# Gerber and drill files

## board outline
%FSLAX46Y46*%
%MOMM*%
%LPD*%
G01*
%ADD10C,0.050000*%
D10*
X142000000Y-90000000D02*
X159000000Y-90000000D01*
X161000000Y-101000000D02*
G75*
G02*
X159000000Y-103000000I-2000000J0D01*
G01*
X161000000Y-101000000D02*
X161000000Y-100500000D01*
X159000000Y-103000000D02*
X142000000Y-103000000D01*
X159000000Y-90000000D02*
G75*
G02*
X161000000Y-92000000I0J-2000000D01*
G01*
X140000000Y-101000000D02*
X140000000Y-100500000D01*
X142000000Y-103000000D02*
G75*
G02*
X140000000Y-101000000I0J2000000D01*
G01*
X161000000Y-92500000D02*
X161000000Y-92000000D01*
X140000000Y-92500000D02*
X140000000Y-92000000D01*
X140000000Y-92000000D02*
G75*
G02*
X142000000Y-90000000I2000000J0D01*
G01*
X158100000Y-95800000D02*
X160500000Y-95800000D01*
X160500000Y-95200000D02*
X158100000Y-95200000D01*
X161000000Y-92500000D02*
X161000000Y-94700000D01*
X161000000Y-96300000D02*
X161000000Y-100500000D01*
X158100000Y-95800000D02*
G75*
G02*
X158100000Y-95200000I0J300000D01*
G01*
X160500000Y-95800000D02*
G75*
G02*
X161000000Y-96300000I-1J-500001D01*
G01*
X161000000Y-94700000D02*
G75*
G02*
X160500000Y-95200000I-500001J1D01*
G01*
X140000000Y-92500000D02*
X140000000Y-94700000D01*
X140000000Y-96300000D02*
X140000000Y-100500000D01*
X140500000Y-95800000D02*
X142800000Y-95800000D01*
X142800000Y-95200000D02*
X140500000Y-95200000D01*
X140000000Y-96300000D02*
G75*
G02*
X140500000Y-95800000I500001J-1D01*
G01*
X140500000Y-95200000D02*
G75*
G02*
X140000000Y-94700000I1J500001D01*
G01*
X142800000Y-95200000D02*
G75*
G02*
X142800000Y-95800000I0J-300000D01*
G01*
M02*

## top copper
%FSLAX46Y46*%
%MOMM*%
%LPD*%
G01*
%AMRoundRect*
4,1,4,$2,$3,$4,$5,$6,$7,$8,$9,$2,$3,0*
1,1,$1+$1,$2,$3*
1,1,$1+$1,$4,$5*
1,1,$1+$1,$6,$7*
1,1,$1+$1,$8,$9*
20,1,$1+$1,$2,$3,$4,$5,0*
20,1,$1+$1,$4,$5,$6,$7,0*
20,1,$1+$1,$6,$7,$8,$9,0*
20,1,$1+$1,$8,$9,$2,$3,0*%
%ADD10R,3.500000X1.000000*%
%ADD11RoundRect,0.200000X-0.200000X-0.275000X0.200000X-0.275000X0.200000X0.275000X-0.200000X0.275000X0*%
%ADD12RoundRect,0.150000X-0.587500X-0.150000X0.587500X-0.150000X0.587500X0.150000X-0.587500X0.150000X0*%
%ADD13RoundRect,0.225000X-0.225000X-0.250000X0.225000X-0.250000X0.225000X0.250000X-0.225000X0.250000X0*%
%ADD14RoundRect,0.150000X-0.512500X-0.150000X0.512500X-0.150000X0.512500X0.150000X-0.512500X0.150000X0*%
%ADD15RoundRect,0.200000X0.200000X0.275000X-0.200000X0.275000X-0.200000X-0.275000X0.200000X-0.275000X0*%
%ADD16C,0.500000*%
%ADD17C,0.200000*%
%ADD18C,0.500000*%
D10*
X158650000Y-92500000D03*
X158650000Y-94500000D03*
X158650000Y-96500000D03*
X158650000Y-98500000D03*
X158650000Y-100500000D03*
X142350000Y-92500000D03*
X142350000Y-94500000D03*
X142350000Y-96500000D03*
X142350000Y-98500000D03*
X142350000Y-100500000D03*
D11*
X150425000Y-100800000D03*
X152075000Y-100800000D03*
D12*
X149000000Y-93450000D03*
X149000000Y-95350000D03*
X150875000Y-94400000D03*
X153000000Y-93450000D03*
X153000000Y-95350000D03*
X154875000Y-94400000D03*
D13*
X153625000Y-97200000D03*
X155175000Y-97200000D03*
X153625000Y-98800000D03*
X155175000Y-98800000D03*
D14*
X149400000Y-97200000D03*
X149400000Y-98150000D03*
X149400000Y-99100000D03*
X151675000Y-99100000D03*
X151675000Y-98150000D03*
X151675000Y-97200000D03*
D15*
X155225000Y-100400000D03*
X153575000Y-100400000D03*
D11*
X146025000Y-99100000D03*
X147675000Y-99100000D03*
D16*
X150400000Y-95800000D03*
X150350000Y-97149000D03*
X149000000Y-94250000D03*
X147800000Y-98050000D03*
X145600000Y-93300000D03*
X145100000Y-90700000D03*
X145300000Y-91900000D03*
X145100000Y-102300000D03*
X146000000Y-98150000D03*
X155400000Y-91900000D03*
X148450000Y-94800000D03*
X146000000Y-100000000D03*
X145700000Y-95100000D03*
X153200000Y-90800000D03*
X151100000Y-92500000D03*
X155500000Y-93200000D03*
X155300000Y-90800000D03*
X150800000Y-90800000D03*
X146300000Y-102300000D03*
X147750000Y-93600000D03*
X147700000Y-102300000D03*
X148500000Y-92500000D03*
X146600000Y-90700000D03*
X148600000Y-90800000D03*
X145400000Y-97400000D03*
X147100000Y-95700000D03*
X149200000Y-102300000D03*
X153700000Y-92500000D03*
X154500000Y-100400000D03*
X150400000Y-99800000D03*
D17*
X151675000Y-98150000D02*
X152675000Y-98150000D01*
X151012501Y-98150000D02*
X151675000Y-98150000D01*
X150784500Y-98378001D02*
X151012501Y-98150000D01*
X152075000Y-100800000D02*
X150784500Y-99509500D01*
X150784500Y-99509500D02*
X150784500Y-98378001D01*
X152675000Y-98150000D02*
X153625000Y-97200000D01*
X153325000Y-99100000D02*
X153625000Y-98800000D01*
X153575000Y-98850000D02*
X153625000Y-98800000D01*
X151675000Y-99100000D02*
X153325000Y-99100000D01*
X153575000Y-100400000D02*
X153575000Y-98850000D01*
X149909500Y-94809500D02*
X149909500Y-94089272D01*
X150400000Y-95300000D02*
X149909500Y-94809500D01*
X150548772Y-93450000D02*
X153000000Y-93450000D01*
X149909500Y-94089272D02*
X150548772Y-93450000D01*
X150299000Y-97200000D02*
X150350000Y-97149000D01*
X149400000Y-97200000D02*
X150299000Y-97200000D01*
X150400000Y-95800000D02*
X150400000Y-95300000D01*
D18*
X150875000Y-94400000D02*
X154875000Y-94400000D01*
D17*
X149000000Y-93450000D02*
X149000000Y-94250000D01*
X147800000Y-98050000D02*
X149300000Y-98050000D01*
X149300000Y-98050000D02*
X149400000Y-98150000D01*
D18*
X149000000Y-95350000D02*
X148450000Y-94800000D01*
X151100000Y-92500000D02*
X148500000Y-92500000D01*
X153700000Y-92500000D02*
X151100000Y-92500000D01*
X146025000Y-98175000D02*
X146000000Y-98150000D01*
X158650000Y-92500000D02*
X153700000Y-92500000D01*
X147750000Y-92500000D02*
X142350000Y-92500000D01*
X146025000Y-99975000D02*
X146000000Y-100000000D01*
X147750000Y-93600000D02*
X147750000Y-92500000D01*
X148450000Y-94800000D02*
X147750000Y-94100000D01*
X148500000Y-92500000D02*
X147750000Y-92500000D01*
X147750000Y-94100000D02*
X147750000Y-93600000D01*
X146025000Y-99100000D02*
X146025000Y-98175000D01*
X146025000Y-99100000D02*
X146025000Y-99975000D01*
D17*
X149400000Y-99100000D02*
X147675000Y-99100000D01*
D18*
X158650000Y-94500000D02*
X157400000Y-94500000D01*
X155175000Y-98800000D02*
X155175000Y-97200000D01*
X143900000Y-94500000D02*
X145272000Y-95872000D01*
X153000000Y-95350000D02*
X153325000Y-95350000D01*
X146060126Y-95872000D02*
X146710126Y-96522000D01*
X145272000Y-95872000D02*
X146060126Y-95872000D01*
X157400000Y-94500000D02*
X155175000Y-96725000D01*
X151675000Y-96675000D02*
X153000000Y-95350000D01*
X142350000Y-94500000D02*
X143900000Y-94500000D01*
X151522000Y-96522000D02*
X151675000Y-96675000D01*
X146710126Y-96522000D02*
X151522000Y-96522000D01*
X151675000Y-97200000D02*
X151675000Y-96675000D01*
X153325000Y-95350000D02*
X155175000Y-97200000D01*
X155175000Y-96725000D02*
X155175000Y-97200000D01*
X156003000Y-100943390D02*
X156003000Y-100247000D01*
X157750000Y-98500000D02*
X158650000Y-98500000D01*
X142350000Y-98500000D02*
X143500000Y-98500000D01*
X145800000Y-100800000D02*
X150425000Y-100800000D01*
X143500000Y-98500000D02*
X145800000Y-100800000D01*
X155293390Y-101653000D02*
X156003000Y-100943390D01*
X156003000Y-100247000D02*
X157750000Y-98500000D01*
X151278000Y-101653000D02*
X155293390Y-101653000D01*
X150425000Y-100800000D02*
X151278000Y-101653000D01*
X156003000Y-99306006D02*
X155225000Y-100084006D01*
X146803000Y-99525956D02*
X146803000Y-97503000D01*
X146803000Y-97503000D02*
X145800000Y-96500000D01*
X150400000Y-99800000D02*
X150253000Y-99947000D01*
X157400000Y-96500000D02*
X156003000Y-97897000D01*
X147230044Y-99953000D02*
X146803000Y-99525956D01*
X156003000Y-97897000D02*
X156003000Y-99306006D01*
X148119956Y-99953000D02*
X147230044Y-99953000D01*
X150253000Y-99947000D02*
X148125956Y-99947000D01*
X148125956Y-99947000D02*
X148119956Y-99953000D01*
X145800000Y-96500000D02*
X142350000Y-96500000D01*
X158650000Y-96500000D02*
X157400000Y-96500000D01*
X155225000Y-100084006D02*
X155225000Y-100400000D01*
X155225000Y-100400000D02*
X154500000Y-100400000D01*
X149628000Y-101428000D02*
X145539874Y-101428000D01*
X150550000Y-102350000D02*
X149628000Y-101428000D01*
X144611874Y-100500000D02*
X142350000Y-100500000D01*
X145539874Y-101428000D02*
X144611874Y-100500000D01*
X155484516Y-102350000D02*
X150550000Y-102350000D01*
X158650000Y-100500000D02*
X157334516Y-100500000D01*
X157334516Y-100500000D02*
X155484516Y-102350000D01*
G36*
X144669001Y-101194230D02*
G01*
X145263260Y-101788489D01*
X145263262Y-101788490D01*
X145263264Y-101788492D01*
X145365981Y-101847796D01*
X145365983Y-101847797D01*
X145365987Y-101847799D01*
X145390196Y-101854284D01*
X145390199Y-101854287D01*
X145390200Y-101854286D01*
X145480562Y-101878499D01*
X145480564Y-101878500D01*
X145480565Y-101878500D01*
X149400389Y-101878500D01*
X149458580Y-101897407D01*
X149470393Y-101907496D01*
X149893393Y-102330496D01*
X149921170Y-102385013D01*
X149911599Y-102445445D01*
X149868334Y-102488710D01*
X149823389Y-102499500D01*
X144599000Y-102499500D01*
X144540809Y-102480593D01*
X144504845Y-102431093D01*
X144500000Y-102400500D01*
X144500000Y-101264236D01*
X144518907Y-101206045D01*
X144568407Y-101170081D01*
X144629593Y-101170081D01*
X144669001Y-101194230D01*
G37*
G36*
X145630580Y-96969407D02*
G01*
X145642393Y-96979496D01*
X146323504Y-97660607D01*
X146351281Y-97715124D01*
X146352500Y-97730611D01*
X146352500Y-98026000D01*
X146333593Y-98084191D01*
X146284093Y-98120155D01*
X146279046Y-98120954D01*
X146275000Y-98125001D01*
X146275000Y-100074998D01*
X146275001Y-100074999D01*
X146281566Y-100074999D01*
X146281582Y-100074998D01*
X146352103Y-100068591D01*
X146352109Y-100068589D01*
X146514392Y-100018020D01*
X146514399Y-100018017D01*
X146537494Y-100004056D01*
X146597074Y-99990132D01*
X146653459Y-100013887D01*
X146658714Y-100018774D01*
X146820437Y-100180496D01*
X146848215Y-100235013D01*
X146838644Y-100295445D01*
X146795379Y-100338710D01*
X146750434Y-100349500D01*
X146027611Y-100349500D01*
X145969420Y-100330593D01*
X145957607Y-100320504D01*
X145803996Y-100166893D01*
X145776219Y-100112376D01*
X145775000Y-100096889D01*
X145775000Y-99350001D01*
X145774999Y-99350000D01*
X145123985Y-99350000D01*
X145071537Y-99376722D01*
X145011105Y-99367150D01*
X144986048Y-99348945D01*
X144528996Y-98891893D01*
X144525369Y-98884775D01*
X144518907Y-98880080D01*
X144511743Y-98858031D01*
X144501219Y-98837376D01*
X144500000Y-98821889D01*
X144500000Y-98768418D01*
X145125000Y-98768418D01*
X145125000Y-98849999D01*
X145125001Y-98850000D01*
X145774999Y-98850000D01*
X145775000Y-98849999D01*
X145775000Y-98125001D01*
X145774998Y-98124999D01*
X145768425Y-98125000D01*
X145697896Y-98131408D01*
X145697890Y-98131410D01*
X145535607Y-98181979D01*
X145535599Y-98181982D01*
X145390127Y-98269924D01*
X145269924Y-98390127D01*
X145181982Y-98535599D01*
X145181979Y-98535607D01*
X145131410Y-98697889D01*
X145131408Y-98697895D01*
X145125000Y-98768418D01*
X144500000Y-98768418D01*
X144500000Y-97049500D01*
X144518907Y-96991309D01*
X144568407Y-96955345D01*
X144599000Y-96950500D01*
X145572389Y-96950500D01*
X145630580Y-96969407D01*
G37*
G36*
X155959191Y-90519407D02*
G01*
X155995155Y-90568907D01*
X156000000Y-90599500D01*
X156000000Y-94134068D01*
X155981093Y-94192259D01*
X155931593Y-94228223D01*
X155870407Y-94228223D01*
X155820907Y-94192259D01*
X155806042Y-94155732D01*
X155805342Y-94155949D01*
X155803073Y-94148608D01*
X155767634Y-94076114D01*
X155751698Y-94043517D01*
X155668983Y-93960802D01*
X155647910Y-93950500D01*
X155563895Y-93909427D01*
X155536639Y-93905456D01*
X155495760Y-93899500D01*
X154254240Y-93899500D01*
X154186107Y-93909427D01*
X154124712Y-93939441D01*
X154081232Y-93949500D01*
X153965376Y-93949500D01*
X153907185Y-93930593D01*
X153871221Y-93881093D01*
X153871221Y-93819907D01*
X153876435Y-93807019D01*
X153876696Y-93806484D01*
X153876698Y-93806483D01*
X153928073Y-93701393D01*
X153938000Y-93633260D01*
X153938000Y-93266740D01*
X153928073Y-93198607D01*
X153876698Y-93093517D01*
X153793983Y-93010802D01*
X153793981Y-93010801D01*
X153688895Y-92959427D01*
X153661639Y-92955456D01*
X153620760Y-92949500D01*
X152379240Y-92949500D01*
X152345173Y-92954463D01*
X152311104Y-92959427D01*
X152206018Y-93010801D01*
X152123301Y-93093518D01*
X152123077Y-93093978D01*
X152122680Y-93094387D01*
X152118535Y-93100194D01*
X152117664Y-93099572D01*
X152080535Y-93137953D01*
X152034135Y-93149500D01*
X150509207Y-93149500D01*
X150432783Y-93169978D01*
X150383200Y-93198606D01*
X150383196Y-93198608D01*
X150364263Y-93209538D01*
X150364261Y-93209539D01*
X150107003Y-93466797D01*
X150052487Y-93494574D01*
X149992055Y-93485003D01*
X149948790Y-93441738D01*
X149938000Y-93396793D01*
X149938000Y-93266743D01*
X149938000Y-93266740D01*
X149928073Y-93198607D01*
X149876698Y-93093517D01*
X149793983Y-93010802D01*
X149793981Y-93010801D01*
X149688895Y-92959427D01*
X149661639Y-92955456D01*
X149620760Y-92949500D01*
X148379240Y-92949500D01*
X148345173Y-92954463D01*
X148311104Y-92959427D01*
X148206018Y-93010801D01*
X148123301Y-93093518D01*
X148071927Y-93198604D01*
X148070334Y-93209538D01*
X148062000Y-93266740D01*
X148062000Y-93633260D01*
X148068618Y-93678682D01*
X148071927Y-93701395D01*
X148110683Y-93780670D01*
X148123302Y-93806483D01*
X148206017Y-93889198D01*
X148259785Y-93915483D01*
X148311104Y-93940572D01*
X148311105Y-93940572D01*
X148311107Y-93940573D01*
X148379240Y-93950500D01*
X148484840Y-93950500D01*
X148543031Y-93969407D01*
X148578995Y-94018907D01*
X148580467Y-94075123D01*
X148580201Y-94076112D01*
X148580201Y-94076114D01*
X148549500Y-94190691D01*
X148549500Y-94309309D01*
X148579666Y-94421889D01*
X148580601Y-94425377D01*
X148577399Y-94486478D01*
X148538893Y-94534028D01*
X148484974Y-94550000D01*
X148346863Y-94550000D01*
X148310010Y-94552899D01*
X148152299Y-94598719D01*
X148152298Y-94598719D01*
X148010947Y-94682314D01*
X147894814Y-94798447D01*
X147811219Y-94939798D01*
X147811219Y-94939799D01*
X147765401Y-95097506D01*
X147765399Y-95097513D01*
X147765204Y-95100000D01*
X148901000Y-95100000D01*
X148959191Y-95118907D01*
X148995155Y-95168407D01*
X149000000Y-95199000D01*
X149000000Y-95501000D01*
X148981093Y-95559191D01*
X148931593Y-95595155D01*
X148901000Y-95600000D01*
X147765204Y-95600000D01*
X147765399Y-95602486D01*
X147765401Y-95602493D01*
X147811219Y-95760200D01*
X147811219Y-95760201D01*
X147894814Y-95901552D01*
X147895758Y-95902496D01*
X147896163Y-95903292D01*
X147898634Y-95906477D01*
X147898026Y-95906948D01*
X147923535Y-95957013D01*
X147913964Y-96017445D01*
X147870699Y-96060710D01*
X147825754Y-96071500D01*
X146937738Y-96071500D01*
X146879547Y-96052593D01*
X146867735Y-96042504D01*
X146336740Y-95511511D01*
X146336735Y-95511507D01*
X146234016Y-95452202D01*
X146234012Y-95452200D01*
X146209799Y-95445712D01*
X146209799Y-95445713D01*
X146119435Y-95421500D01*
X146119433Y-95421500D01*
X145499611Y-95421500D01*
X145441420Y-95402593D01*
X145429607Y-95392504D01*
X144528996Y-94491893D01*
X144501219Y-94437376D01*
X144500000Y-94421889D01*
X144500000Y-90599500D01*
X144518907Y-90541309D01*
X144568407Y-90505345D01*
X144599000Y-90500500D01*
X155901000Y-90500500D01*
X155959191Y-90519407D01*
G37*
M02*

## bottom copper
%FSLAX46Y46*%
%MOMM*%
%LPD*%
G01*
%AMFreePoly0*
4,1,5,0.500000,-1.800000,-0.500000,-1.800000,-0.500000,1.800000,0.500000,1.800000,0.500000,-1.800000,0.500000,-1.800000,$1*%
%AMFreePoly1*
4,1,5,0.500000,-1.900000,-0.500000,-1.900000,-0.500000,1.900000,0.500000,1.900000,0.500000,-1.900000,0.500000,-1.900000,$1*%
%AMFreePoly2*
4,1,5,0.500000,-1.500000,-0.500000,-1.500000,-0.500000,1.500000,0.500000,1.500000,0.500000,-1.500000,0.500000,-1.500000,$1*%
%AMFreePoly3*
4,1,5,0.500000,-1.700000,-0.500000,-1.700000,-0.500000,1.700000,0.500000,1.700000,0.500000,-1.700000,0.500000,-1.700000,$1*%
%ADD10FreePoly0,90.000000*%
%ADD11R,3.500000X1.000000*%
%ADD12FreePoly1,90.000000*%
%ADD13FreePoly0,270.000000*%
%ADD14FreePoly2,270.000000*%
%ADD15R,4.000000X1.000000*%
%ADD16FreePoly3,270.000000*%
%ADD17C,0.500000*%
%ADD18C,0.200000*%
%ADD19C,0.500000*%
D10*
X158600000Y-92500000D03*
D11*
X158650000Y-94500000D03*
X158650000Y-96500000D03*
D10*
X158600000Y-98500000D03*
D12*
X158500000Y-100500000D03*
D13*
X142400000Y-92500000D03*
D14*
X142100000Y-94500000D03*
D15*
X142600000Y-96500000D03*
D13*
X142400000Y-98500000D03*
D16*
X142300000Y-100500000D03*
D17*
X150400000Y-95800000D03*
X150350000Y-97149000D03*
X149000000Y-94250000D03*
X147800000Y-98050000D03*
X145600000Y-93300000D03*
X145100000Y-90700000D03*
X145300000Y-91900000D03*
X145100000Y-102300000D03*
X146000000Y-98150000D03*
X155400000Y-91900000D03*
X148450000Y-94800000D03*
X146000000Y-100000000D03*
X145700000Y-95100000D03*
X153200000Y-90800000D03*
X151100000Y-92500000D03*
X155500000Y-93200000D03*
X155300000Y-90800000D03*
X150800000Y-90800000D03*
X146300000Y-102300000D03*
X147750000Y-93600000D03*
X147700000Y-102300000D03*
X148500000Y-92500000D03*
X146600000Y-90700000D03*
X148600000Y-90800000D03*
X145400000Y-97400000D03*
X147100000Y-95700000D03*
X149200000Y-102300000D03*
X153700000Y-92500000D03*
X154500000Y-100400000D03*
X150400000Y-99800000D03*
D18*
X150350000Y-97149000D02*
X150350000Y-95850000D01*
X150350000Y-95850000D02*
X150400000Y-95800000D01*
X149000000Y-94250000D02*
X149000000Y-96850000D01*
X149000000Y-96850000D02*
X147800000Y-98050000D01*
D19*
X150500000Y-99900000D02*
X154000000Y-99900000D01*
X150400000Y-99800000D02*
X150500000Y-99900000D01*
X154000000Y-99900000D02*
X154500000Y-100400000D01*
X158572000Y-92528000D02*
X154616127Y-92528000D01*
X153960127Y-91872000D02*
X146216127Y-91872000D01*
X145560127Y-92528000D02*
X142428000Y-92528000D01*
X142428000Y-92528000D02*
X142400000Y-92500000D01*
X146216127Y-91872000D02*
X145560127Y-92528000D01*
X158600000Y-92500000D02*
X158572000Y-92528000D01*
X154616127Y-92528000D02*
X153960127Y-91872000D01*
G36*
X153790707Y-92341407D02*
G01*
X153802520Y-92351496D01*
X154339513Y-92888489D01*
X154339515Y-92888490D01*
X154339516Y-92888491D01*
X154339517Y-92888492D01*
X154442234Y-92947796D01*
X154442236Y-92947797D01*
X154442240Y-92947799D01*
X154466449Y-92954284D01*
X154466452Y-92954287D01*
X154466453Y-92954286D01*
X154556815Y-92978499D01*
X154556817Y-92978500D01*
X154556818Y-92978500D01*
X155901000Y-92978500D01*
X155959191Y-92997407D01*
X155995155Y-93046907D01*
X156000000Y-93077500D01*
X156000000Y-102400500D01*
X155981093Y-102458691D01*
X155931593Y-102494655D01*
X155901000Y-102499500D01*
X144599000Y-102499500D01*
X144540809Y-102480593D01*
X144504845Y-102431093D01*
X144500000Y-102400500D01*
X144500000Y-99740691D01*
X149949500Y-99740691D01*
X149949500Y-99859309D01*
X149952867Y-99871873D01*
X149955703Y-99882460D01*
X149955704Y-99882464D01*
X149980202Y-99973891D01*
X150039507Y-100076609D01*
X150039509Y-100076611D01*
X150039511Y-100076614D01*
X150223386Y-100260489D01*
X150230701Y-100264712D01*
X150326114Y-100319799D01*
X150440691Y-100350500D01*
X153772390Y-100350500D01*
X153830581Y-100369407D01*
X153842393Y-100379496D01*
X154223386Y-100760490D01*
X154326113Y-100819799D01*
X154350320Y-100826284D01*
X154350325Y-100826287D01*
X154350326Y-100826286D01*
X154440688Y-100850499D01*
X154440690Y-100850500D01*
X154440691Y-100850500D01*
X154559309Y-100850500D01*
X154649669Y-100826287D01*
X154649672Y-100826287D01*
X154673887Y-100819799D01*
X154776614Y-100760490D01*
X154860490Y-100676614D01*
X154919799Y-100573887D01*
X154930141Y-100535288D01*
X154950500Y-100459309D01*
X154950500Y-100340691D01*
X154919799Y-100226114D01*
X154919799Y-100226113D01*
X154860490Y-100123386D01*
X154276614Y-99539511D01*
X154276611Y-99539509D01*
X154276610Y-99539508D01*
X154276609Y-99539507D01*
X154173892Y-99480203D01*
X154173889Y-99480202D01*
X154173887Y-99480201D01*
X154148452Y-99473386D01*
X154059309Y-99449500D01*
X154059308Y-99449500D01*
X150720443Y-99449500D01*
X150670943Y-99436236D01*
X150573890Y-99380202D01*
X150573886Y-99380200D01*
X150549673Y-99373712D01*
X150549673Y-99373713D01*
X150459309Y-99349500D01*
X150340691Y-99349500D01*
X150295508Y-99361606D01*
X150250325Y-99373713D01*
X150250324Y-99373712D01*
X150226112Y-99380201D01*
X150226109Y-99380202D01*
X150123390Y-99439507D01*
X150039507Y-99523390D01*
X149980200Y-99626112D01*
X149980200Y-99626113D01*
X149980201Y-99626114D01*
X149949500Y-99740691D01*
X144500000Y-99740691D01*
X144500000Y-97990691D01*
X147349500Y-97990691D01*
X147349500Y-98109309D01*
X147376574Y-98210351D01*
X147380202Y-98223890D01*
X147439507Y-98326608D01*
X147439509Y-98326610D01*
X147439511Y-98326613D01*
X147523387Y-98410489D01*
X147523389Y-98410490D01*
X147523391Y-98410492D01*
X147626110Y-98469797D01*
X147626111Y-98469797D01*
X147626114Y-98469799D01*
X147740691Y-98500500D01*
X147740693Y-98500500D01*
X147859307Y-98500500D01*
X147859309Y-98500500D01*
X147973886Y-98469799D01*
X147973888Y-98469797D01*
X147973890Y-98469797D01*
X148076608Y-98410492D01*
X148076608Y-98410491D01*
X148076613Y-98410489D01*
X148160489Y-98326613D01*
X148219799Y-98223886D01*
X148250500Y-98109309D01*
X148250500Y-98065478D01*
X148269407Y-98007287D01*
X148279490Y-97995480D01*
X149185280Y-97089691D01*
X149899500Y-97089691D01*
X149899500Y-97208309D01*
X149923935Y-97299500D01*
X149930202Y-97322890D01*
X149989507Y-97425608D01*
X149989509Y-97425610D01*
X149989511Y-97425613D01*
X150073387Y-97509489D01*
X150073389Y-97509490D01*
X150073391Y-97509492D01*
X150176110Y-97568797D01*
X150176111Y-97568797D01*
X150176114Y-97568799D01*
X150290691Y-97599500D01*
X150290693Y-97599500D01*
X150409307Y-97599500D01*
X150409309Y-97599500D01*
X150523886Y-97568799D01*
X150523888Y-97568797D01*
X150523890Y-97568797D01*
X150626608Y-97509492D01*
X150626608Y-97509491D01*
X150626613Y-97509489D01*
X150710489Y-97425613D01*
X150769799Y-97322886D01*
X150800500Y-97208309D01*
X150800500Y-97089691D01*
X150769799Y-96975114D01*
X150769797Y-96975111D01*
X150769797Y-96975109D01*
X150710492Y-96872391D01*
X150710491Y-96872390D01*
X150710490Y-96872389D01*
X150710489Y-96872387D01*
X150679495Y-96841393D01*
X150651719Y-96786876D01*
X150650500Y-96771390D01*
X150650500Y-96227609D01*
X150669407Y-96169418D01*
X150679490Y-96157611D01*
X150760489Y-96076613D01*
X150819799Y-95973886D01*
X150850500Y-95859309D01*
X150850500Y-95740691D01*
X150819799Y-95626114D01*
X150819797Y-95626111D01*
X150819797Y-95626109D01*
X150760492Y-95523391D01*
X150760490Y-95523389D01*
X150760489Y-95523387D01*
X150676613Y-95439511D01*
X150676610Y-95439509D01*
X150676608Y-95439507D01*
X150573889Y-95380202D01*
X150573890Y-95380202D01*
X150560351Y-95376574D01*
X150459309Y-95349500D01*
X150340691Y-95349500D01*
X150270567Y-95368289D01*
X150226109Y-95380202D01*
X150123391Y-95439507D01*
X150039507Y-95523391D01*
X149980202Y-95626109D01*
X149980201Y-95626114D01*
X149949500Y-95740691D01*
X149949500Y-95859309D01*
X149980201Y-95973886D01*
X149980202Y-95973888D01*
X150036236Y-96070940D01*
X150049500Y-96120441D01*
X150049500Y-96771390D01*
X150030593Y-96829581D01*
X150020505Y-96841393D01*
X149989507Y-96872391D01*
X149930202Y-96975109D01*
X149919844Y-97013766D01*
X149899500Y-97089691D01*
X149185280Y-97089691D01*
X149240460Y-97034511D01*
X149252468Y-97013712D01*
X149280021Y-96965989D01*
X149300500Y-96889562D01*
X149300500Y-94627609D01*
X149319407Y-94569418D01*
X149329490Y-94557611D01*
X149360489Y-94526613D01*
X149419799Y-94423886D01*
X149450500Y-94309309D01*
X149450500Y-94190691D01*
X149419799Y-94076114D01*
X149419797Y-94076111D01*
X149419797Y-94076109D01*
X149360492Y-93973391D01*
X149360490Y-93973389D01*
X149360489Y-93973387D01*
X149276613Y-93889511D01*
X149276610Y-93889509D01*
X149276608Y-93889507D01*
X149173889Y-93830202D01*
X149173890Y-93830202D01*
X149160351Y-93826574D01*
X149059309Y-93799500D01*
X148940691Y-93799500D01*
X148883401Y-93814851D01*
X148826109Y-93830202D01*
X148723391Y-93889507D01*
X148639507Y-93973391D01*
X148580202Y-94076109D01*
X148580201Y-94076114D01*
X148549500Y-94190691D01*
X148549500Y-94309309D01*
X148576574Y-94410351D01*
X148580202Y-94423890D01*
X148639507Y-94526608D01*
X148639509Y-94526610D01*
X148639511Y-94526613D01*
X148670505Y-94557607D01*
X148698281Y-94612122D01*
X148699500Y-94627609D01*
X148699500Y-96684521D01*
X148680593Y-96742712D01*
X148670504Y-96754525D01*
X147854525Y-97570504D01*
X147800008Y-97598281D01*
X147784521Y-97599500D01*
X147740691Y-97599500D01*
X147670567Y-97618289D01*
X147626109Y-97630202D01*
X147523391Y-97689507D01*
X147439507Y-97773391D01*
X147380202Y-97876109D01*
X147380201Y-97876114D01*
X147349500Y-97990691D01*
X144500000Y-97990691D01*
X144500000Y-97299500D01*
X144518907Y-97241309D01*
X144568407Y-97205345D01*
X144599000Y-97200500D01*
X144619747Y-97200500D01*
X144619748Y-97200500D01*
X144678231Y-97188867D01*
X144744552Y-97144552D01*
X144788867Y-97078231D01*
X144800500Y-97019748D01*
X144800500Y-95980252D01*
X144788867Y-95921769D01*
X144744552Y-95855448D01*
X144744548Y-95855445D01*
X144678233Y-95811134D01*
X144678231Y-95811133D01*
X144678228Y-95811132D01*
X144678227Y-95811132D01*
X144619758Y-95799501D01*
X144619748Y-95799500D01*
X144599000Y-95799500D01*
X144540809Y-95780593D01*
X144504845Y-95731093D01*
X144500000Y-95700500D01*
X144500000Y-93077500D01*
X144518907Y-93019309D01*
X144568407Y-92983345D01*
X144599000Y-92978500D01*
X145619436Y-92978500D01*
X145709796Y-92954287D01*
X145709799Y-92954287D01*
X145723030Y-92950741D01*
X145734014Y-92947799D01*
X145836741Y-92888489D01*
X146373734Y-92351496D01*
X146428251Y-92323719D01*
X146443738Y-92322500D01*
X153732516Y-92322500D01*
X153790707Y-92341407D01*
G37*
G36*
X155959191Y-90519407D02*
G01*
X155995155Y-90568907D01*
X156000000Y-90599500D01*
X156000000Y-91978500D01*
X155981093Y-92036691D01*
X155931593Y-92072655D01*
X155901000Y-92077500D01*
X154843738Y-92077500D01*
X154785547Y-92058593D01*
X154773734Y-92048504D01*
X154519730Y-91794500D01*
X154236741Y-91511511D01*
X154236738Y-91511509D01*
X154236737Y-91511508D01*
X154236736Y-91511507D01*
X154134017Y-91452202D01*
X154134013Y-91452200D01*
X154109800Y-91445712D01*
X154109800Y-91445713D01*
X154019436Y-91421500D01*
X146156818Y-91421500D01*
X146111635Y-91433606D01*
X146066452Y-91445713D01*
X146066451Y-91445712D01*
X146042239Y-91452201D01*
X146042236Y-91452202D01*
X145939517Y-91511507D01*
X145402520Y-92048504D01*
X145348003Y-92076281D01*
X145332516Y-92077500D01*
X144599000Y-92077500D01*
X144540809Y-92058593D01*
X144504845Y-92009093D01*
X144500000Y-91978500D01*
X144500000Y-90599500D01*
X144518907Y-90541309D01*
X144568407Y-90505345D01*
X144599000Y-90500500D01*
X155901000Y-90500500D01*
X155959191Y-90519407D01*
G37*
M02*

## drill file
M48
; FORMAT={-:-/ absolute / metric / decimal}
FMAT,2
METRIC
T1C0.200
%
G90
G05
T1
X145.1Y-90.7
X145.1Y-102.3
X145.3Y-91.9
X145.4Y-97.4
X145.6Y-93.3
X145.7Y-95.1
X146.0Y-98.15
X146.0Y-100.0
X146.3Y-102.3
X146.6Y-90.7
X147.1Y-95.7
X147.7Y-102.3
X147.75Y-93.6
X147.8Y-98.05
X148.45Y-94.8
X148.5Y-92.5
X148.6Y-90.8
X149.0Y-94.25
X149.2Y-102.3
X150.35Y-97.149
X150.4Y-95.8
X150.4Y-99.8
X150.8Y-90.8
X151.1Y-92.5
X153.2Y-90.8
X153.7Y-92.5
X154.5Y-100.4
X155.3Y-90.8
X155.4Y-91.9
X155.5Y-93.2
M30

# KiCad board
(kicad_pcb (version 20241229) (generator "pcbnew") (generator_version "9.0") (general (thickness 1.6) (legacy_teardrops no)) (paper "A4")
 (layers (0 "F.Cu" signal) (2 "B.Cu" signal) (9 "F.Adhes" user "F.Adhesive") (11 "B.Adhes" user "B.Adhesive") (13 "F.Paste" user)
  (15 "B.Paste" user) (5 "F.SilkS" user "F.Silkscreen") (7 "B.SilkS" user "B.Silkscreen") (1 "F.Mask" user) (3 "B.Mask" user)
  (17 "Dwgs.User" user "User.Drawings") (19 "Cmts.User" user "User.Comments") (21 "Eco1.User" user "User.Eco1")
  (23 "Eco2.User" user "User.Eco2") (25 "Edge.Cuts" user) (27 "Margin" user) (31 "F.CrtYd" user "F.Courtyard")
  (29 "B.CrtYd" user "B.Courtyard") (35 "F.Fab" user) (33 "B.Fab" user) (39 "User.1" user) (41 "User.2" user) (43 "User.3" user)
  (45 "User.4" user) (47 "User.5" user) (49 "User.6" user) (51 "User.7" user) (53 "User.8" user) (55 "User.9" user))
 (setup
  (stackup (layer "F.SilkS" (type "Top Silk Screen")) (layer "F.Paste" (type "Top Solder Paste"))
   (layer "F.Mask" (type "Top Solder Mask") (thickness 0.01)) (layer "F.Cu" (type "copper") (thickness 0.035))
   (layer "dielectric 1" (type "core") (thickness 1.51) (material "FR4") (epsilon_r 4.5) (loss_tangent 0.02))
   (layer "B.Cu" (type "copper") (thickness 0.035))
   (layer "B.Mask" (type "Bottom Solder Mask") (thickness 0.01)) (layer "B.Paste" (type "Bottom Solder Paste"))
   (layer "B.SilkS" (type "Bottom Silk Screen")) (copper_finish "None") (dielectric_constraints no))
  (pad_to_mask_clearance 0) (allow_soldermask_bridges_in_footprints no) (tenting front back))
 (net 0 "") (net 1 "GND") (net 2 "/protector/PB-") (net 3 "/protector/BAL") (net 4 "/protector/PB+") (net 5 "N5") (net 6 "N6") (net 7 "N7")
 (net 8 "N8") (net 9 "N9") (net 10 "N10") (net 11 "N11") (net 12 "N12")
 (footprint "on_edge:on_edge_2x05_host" (layer "F.Cu") (at 161 96.5 -90)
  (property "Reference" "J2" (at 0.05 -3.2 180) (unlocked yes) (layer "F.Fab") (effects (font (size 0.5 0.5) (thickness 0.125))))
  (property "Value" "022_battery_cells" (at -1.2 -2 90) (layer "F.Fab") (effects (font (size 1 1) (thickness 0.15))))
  (fp_line (start -0.7 2.9) (end -0.7 0.5) (stroke (width 0.05) (type solid)) (layer "Edge.Cuts"))
  (fp_line (start -1.3 0.5) (end -1.3 2.9) (stroke (width 0.05) (type solid)) (layer "Edge.Cuts"))
  (fp_line (start -4 0) (end -1.8 0) (stroke (width 0.05) (type solid)) (layer "Edge.Cuts"))
  (fp_line (start -0.2 0) (end 4 0) (stroke (width 0.05) (type solid)) (layer "Edge.Cuts"))
  (fp_arc (start -0.7 2.9) (mid -1 3.2) (end -1.3 2.9) (stroke (width 0.05) (type solid)) (layer "Edge.Cuts"))
  (fp_arc (start -0.7 0.5) (mid -0.553553 0.146447) (end -0.2 0) (stroke (width 0.05) (type solid)) (layer "Edge.Cuts"))
  (fp_arc (start -1.8 0) (mid -1.446447 0.146447) (end -1.3 0.5) (stroke (width 0.05) (type solid)) (layer "Edge.Cuts"))
  (pad "1" smd rect (at -4 2.35 270) (size 1 3.5) (layers "F.Cu" "F.Mask") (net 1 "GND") (zone_connect 0))
  (pad "2" smd rect (at -2 2.35 270) (size 1 3.5) (layers "F.Cu" "F.Mask") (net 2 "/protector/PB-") (zone_connect 0))
  (pad "3" smd rect (at 0 2.35 270) (size 1 3.5) (layers "F.Cu" "F.Mask") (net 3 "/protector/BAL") (zone_connect 0))
  (pad "4" smd rect (at 2 2.35 270) (size 1 3.5) (layers "F.Cu" "F.Mask") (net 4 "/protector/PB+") (zone_connect 0))
  (pad "5" smd rect (at 4 2.35 270) (size 1 3.5) (layers "F.Cu" "F.Mask") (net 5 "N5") (zone_connect 0))
  (pad "6" smd custom (at -4 2.4 90) (size 1 3.6) (layers "B.Cu" "B.Mask") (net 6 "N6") (zone_connect 0)
   (options (clearance outline) (anchor rect)) (primitives))
  (pad "7" smd rect (at -2 2.35 90) (size 1 3.5) (layers "B.Cu" "B.Mask") (zone_connect 0))
  (pad "8" smd rect (at 0 2.35 90) (size 1 3.5) (layers "B.Cu" "B.Mask") (zone_connect 0))
  (pad "9" smd custom (at 2 2.4 90) (size 1 3.6) (layers "B.Cu" "B.Mask") (zone_connect 0) (options (clearance outline) (anchor rect))
   (primitives))
  (pad "10" smd custom (at 4 2.5 90) (size 1 3.8) (layers "B.Cu" "B.Mask") (zone_connect 0) (options (clearance outline) (anchor rect))
   (primitives))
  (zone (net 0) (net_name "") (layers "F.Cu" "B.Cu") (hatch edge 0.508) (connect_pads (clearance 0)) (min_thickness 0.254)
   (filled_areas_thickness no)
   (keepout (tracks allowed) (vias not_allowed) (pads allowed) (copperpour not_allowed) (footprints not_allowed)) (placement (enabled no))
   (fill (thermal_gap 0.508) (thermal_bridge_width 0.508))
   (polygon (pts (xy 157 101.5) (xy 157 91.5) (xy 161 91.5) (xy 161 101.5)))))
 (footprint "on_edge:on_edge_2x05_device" (layer "F.Cu") (at 140 96.5 -90)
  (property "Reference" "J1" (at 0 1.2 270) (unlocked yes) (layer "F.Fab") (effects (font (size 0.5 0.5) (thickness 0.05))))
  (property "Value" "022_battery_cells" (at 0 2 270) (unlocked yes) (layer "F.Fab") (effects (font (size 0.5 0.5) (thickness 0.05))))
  (fp_line (start -4 0) (end -1.8 0) (stroke (width 0.05) (type solid)) (layer "Edge.Cuts"))
  (fp_line (start -0.2 0) (end 4 0) (stroke (width 0.05) (type solid)) (layer "Edge.Cuts"))
  (fp_line (start -0.7 -0.5) (end -0.7 -2.8) (stroke (width 0.05) (type solid)) (layer "Edge.Cuts"))
  (fp_line (start -1.3 -2.8) (end -1.3 -0.5) (stroke (width 0.05) (type solid)) (layer "Edge.Cuts"))
  (fp_arc (start -0.2 0) (mid -0.553553 -0.146447) (end -0.7 -0.5) (stroke (width 0.05) (type solid)) (layer "Edge.Cuts"))
  (fp_arc (start -1.3 -0.5) (mid -1.446447 -0.146447) (end -1.8 0) (stroke (width 0.05) (type solid)) (layer "Edge.Cuts"))
  (fp_arc (start -1.3 -2.8) (mid -1 -3.1) (end -0.7 -2.8) (stroke (width 0.05) (type solid)) (layer "Edge.Cuts"))
  (pad "1" smd rect (at -4 -2.35 90) (size 1 3.5) (layers "F.Cu" "F.Mask") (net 1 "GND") (zone_connect 0))
  (pad "2" smd rect (at -2 -2.35 270) (size 1 3.5) (layers "F.Cu" "F.Mask") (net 2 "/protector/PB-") (zone_connect 0))
  (pad "3" smd rect (at 0 -2.35 270) (size 1 3.5) (layers "F.Cu" "F.Mask") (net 3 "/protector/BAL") (zone_connect 0))
  (pad "4" smd rect (at 2 -2.35 90) (size 1 3.5) (layers "F.Cu" "F.Mask") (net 4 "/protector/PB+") (zone_connect 0))
  (pad "5" smd rect (at 4 -2.35 90) (size 1 3.5) (layers "F.Cu" "F.Mask") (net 5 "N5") (zone_connect 0))
  (pad "6" smd custom (at -4 -2.4 270) (size 1 3.6) (layers "B.Cu" "B.Mask") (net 6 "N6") (zone_connect 0)
   (options (clearance outline) (anchor rect)) (primitives))
  (pad "7" smd custom (at -2 -2.1 270) (size 1 3) (layers "B.Cu" "B.Mask") (zone_connect 0) (options (clearance outline) (anchor rect))
   (primitives))
  (pad "8" smd rect (at 0 -2.6 270) (size 1 4) (layers "B.Cu" "B.Mask") (zone_connect 0))
  (pad "9" smd custom (at 2 -2.4 270) (size 1 3.6) (layers "B.Cu" "B.Mask") (zone_connect 0) (options (clearance outline) (anchor rect))
   (primitives))
  (pad "10" smd custom (at 4 -2.3 270) (size 1 3.4) (layers "B.Cu" "B.Mask") (zone_connect 0) (options (clearance outline) (anchor rect))
   (primitives))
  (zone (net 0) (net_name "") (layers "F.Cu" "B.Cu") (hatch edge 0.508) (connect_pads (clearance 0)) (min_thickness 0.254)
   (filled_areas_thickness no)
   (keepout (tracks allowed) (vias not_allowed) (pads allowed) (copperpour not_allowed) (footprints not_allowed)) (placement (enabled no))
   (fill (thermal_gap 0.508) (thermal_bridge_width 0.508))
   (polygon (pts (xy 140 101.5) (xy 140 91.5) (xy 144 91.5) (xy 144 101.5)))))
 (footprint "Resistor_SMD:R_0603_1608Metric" (layer "F.Cu") (at 151.25 100.8)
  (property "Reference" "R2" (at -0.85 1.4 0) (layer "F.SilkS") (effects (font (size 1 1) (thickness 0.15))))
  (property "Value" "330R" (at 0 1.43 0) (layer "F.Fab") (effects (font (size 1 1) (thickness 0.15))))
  (pad "1" smd roundrect (at -0.825 0) (size 0.8 0.95) (layers "F.Cu" "F.Mask" "F.Paste") (roundrect_rratio 0.25) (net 4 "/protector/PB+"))
  (pad "2" smd roundrect (at 0.825 0) (size 0.8 0.95) (layers "F.Cu" "F.Mask" "F.Paste") (roundrect_rratio 0.25) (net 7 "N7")))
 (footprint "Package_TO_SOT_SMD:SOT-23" (layer "F.Cu") (at 149.9375 94.4)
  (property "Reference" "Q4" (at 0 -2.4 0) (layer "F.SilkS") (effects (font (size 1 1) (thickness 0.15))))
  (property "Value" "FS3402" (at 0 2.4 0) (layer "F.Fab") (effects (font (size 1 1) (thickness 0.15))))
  (pad "1" smd roundrect (at -0.9375 -0.95) (size 1.475 0.6) (layers "F.Cu" "F.Mask" "F.Paste") (roundrect_rratio 0.25) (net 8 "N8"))
  (pad "2" smd roundrect (at -0.9375 0.95) (size 1.475 0.6) (layers "F.Cu" "F.Mask" "F.Paste") (roundrect_rratio 0.25) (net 1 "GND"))
  (pad "3" smd roundrect (at 0.9375 0) (size 1.475 0.6) (layers "F.Cu" "F.Mask" "F.Paste") (roundrect_rratio 0.25) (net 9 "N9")))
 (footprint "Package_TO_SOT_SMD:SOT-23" (layer "F.Cu") (at 153.9375 94.4)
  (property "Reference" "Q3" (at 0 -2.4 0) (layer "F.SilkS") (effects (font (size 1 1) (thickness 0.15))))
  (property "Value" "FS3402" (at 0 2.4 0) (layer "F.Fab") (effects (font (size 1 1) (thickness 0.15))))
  (pad "1" smd roundrect (at -0.9375 -0.95) (size 1.475 0.6) (layers "F.Cu" "F.Mask" "F.Paste") (roundrect_rratio 0.25) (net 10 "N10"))
  (pad "2" smd roundrect (at -0.9375 0.95) (size 1.475 0.6) (layers "F.Cu" "F.Mask" "F.Paste") (roundrect_rratio 0.25)
   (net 2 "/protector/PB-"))
  (pad "3" smd roundrect (at 0.9375 0) (size 1.475 0.6) (layers "F.Cu" "F.Mask" "F.Paste") (roundrect_rratio 0.25) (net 9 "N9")))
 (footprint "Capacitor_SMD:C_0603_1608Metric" (layer "F.Cu") (at 154.4 97.2)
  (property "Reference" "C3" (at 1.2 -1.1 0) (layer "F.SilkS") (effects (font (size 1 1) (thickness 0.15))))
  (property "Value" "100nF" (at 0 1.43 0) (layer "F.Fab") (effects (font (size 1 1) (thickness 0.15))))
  (pad "1" smd roundrect (at -0.775 0) (size 0.9 0.95) (layers "F.Cu" "F.Mask" "F.Paste") (roundrect_rratio 0.25) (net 7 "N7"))
  (pad "2" smd roundrect (at 0.775 0) (size 0.9 0.95) (layers "F.Cu" "F.Mask" "F.Paste") (roundrect_rratio 0.25) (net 2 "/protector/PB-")))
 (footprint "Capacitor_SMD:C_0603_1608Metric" (layer "F.Cu") (at 154.4 98.8)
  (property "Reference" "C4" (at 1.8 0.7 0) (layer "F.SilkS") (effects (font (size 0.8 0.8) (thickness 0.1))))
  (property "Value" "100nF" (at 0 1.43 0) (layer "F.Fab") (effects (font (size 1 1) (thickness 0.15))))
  (pad "1" smd roundrect (at -0.775 0) (size 0.9 0.95) (layers "F.Cu" "F.Mask" "F.Paste") (roundrect_rratio 0.25) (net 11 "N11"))
  (pad "2" smd roundrect (at 0.775 0) (size 0.9 0.95) (layers "F.Cu" "F.Mask" "F.Paste") (roundrect_rratio 0.25) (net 2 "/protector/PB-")))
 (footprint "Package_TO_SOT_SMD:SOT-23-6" (layer "F.Cu") (at 150.5375 98.15)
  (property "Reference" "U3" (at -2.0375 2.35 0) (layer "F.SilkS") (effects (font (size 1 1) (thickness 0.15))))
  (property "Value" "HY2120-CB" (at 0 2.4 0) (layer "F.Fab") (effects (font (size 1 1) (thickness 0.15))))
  (pad "1" smd roundrect (at -1.1375 -0.95) (size 1.325 0.6) (layers "F.Cu" "F.Mask" "F.Paste") (roundrect_rratio 0.25) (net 10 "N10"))
  (pad "2" smd roundrect (at -1.1375 0) (size 1.325 0.6) (layers "F.Cu" "F.Mask" "F.Paste") (roundrect_rratio 0.25) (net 8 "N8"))
  (pad "3" smd roundrect (at -1.1375 0.95) (size 1.325 0.6) (layers "F.Cu" "F.Mask" "F.Paste") (roundrect_rratio 0.25) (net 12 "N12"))
  (pad "4" smd roundrect (at 1.1375 0.95) (size 1.325 0.6) (layers "F.Cu" "F.Mask" "F.Paste") (roundrect_rratio 0.25) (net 11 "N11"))
  (pad "5" smd roundrect (at 1.1375 0) (size 1.325 0.6) (layers "F.Cu" "F.Mask" "F.Paste") (roundrect_rratio 0.25) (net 7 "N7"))
  (pad "6" smd roundrect (at 1.1375 -0.95) (size 1.325 0.6) (layers "F.Cu" "F.Mask" "F.Paste") (roundrect_rratio 0.25)
   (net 2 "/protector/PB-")))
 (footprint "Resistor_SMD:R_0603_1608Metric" (layer "F.Cu") (at 154.4 100.4 180)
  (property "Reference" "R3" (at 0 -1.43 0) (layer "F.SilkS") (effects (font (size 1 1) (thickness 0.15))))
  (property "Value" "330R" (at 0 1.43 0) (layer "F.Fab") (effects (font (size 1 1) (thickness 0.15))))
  (pad "1" smd roundrect (at -0.825 0 180) (size 0.8 0.95) (layers "F.Cu" "F.Mask" "F.Paste") (roundrect_rratio 0.25)
   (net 3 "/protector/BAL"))
  (pad "2" smd roundrect (at 0.825 0 180) (size 0.8 0.95) (layers "F.Cu" "F.Mask" "F.Paste") (roundrect_rratio 0.25) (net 11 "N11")))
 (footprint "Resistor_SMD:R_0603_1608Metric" (layer "F.Cu") (at 146.85 99.1)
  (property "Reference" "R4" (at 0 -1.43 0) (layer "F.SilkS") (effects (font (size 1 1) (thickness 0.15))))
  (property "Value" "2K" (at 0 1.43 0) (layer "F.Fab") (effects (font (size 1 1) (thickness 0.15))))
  (pad "1" smd roundrect (at -0.825 0) (size 0.8 0.95) (layers "F.Cu" "F.Mask" "F.Paste") (roundrect_rratio 0.25) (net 1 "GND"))
  (pad "2" smd roundrect (at 0.825 0) (size 0.8 0.95) (layers "F.Cu" "F.Mask" "F.Paste") (roundrect_rratio 0.25) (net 12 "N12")))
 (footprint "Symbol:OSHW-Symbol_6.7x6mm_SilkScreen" (layer "B.Cu") (at 149.175 95.9 180)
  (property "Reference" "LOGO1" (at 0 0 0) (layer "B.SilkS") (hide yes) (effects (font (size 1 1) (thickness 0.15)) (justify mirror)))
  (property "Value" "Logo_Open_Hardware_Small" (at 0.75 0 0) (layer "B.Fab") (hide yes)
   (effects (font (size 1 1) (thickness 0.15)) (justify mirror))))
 (gr_line (start 142 90) (end 159 90) (stroke (width 0.05) (type solid)) (layer "Edge.Cuts"))
 (gr_arc (start 161 101) (mid 160.414214 102.414214) (end 159 103) (stroke (width 0.05) (type solid)) (layer "Edge.Cuts"))
 (gr_line (start 161 101) (end 161 100.5) (stroke (width 0.05) (type solid)) (layer "Edge.Cuts"))
 (gr_line (start 159 103) (end 142 103) (stroke (width 0.05) (type solid)) (layer "Edge.Cuts"))
 (gr_arc (start 159 90) (mid 160.414214 90.585786) (end 161 92) (stroke (width 0.05) (type solid)) (layer "Edge.Cuts"))
 (gr_line (start 140 101) (end 140 100.5) (stroke (width 0.05) (type solid)) (layer "Edge.Cuts"))
 (gr_arc (start 142 103) (mid 140.585786 102.414214) (end 140 101) (stroke (width 0.05) (type solid)) (layer "Edge.Cuts"))
 (gr_line (start 161 92.5) (end 161 92) (stroke (width 0.05) (type solid)) (layer "Edge.Cuts"))
 (gr_line (start 140 92.5) (end 140 92) (stroke (width 0.05) (type solid)) (layer "Edge.Cuts"))
 (gr_arc (start 140 92) (mid 140.585786 90.585786) (end 142 90) (stroke (width 0.05) (type solid)) (layer "Edge.Cuts"))
 (segment (start 151.675 98.15) (end 152.675 98.15) (width 0.2) (layer "F.Cu") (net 7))
 (segment (start 151.012501 98.15) (end 151.675 98.15) (width 0.2) (layer "F.Cu") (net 7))
 (segment (start 150.7845 98.378001) (end 151.012501 98.15) (width 0.2) (layer "F.Cu") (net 7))
 (segment (start 152.075 100.8) (end 150.7845 99.5095) (width 0.2) (layer "F.Cu") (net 7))
 (segment (start 150.7845 99.5095) (end 150.7845 98.378001) (width 0.2) (layer "F.Cu") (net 7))
 (segment (start 152.675 98.15) (end 153.625 97.2) (width 0.2) (layer "F.Cu") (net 7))
 (segment (start 153.325 99.1) (end 153.625 98.8) (width 0.2) (layer "F.Cu") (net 11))
 (segment (start 153.575 98.85) (end 153.625 98.8) (width 0.2) (layer "F.Cu") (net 11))
 (segment (start 151.675 99.1) (end 153.325 99.1) (width 0.2) (layer "F.Cu") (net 11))
 (segment (start 153.575 100.4) (end 153.575 98.85) (width 0.2) (layer "F.Cu") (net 11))
 (segment (start 149.9095 94.8095) (end 149.9095 94.089272) (width 0.2) (layer "F.Cu") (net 10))
 (segment (start 150.4 95.3) (end 149.9095 94.8095) (width 0.2) (layer "F.Cu") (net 10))
 (segment (start 150.548772 93.45) (end 153 93.45) (width 0.2) (layer "F.Cu") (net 10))
 (segment (start 149.9095 94.089272) (end 150.548772 93.45) (width 0.2) (layer "F.Cu") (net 10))
 (segment (start 150.299 97.2) (end 150.35 97.149) (width 0.2) (layer "F.Cu") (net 10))
 (segment (start 149.4 97.2) (end 150.299 97.2) (width 0.2) (layer "F.Cu") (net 10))
 (segment (start 150.4 95.8) (end 150.4 95.3) (width 0.2) (layer "F.Cu") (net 10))
 (via (at 150.4 95.8) (size 0.5) (drill 0.2) (layers "F.Cu" "B.Cu") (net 10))
 (via (at 150.35 97.149) (size 0.5) (drill 0.2) (layers "F.Cu" "B.Cu") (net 10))
 (segment (start 150.35 97.149) (end 150.35 95.85) (width 0.2) (layer "B.Cu") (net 10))
 (segment (start 150.35 95.85) (end 150.4 95.8) (width 0.2) (layer "B.Cu") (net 10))
 (segment (start 150.875 94.4) (end 154.875 94.4) (width 0.5) (layer "F.Cu") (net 9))
 (segment (start 149 93.45) (end 149 94.25) (width 0.2) (layer "F.Cu") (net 8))
 (segment (start 147.8 98.05) (end 149.3 98.05) (width 0.2) (layer "F.Cu") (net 8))
 (segment (start 149.3 98.05) (end 149.4 98.15) (width 0.2) (layer "F.Cu") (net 8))
 (via (at 149 94.25) (size 0.5) (drill 0.2) (layers "F.Cu" "B.Cu") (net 8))
 (via (at 147.8 98.05) (size 0.5) (drill 0.2) (layers "F.Cu" "B.Cu") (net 8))
 (segment (start 149 94.25) (end 149 96.85) (width 0.2) (layer "B.Cu") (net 8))
 (segment (start 149 96.85) (end 147.8 98.05) (width 0.2) (layer "B.Cu") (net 8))
 (segment (start 149 95.35) (end 148.45 94.8) (width 0.5) (layer "F.Cu") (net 1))
 (segment (start 151.1 92.5) (end 148.5 92.5) (width 0.5) (layer "F.Cu") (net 1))
 (segment (start 153.7 92.5) (end 151.1 92.5) (width 0.5) (layer "F.Cu") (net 1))
 (segment (start 146.025 98.175) (end 146 98.15) (width 0.5) (layer "F.Cu") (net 1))
 (segment (start 158.65 92.5) (end 153.7 92.5) (width 0.5) (layer "F.Cu") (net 1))
 (segment (start 147.75 92.5) (end 142.35 92.5) (width 0.5) (layer "F.Cu") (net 1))
 (segment (start 146.025 99.975) (end 146 100) (width 0.5) (layer "F.Cu") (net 1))
 (segment (start 147.75 93.6) (end 147.75 92.5) (width 0.5) (layer "F.Cu") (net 1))
 (segment (start 148.45 94.8) (end 147.75 94.1) (width 0.5) (layer "F.Cu") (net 1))
 (segment (start 148.5 92.5) (end 147.75 92.5) (width 0.5) (layer "F.Cu") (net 1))
 (segment (start 147.75 94.1) (end 147.75 93.6) (width 0.5) (layer "F.Cu") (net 1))
 (segment (start 146.025 99.1) (end 146.025 98.175) (width 0.5) (layer "F.Cu") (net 1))
 (segment (start 146.025 99.1) (end 146.025 99.975) (width 0.5) (layer "F.Cu") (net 1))
 (via (at 145.6 93.3) (size 0.5) (drill 0.2) (layers "F.Cu" "B.Cu") (free yes) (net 1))
 (via (at 145.1 90.7) (size 0.5) (drill 0.2) (layers "F.Cu" "B.Cu") (free yes) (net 1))
 (via (at 145.3 91.9) (size 0.5) (drill 0.2) (layers "F.Cu" "B.Cu") (free yes) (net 1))
 (via (at 145.1 102.3) (size 0.5) (drill 0.2) (layers "F.Cu" "B.Cu") (free yes) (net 1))
 (via (at 146 98.15) (size 0.5) (drill 0.2) (layers "F.Cu" "B.Cu") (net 1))
 (via (at 155.4 91.9) (size 0.5) (drill 0.2) (layers "F.Cu" "B.Cu") (free yes) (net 1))
 (via (at 148.45 94.8) (size 0.5) (drill 0.2) (layers "F.Cu" "B.Cu") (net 1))
 (via (at 146 100) (size 0.5) (drill 0.2) (layers "F.Cu" "B.Cu") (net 1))
 (via (at 145.7 95.1) (size 0.5) (drill 0.2) (layers "F.Cu" "B.Cu") (free yes) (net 1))
 (via (at 153.2 90.8) (size 0.5) (drill 0.2) (layers "F.Cu" "B.Cu") (free yes) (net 1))
 (via (at 151.1 92.5) (size 0.5) (drill 0.2) (layers "F.Cu" "B.Cu") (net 1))
 (via (at 155.5 93.2) (size 0.5) (drill 0.2) (layers "F.Cu" "B.Cu") (free yes) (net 1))
 (via (at 155.3 90.8) (size 0.5) (drill 0.2) (layers "F.Cu" "B.Cu") (free yes) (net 1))
 (via (at 150.8 90.8) (size 0.5) (drill 0.2) (layers "F.Cu" "B.Cu") (free yes) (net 1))
 (via (at 146.3 102.3) (size 0.5) (drill 0.2) (layers "F.Cu" "B.Cu") (free yes) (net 1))
 (via (at 147.75 93.6) (size 0.5) (drill 0.2) (layers "F.Cu" "B.Cu") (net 1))
 (via (at 147.7 102.3) (size 0.5) (drill 0.2) (layers "F.Cu" "B.Cu") (free yes) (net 1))
 (via (at 148.5 92.5) (size 0.5) (drill 0.2) (layers "F.Cu" "B.Cu") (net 1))
 (via (at 146.6 90.7) (size 0.5) (drill 0.2) (layers "F.Cu" "B.Cu") (free yes) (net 1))
 (via (at 148.6 90.8) (size 0.5) (drill 0.2) (layers "F.Cu" "B.Cu") (free yes) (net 1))
 (via (at 145.4 97.4) (size 0.5) (drill 0.2) (layers "F.Cu" "B.Cu") (free yes) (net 1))
 (via (at 147.1 95.7) (size 0.5) (drill 0.2) (layers "F.Cu" "B.Cu") (free yes) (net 1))
 (via (at 149.2 102.3) (size 0.5) (drill 0.2) (layers "F.Cu" "B.Cu") (free yes) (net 1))
 (via (at 153.7 92.5) (size 0.5) (drill 0.2) (layers "F.Cu" "B.Cu") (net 1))
 (segment (start 149.4 99.1) (end 147.675 99.1) (width 0.2) (layer "F.Cu") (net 12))
 (segment (start 158.65 94.5) (end 157.4 94.5) (width 0.5) (layer "F.Cu") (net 2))
 (segment (start 155.175 98.8) (end 155.175 97.2) (width 0.5) (layer "F.Cu") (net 2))
 (segment (start 143.9 94.5) (end 145.272 95.872) (width 0.5) (layer "F.Cu") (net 2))
 (segment (start 153 95.35) (end 153.325 95.35) (width 0.5) (layer "F.Cu") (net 2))
 (segment (start 146.060126 95.872) (end 146.710126 96.522) (width 0.5) (layer "F.Cu") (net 2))
 (segment (start 145.272 95.872) (end 146.060126 95.872) (width 0.5) (layer "F.Cu") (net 2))
 (segment (start 157.4 94.5) (end 155.175 96.725) (width 0.5) (layer "F.Cu") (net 2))
 (segment (start 151.675 96.675) (end 153 95.35) (width 0.5) (layer "F.Cu") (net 2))
 (segment (start 142.35 94.5) (end 143.9 94.5) (width 0.5) (layer "F.Cu") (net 2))
 (segment (start 151.522 96.522) (end 151.675 96.675) (width 0.5) (layer "F.Cu") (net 2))
 (segment (start 146.710126 96.522) (end 151.522 96.522) (width 0.5) (layer "F.Cu") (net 2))
 (segment (start 151.675 97.2) (end 151.675 96.675) (width 0.5) (layer "F.Cu") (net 2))
 (segment (start 153.325 95.35) (end 155.175 97.2) (width 0.5) (layer "F.Cu") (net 2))
 (segment (start 155.175 96.725) (end 155.175 97.2) (width 0.5) (layer "F.Cu") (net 2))
 (segment (start 156.003 100.94339) (end 156.003 100.247) (width 0.5) (layer "F.Cu") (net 4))
 (segment (start 157.75 98.5) (end 158.65 98.5) (width 0.5) (layer "F.Cu") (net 4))
 (segment (start 142.35 98.5) (end 143.5 98.5) (width 0.5) (layer "F.Cu") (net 4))
 (segment (start 145.8 100.8) (end 150.425 100.8) (width 0.5) (layer "F.Cu") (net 4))
 (segment (start 143.5 98.5) (end 145.8 100.8) (width 0.5) (layer "F.Cu") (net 4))
 (segment (start 155.29339 101.653) (end 156.003 100.94339) (width 0.5) (layer "F.Cu") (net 4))
 (segment (start 156.003 100.247) (end 157.75 98.5) (width 0.5) (layer "F.Cu") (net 4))
 (segment (start 151.278 101.653) (end 155.29339 101.653) (width 0.5) (layer "F.Cu") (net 4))
 (segment (start 150.425 100.8) (end 151.278 101.653) (width 0.5) (layer "F.Cu") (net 4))
 (segment (start 156.003 99.306006) (end 155.225 100.084006) (width 0.5) (layer "F.Cu") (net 3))
 (segment (start 146.803 99.525956) (end 146.803 97.503) (width 0.5) (layer "F.Cu") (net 3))
 (segment (start 146.803 97.503) (end 145.8 96.5) (width 0.5) (layer "F.Cu") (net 3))
 (segment (start 150.4 99.8) (end 150.253 99.947) (width 0.5) (layer "F.Cu") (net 3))
 (segment (start 157.4 96.5) (end 156.003 97.897) (width 0.5) (layer "F.Cu") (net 3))
 (segment (start 147.230044 99.953) (end 146.803 99.525956) (width 0.5) (layer "F.Cu") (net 3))
 (segment (start 156.003 97.897) (end 156.003 99.306006) (width 0.5) (layer "F.Cu") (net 3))
 (segment (start 148.119956 99.953) (end 147.230044 99.953) (width 0.5) (layer "F.Cu") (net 3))
 (segment (start 150.253 99.947) (end 148.125956 99.947) (width 0.5) (layer "F.Cu") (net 3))
 (segment (start 148.125956 99.947) (end 148.119956 99.953) (width 0.5) (layer "F.Cu") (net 3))
 (segment (start 145.8 96.5) (end 142.35 96.5) (width 0.5) (layer "F.Cu") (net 3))
 (segment (start 158.65 96.5) (end 157.4 96.5) (width 0.5) (layer "F.Cu") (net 3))
 (segment (start 155.225 100.084006) (end 155.225 100.4) (width 0.5) (layer "F.Cu") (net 3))
 (segment (start 155.225 100.4) (end 154.5 100.4) (width 0.5) (layer "F.Cu") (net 3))
 (via (at 154.5 100.4) (size 0.5) (drill 0.2) (layers "F.Cu" "B.Cu") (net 3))
 (via (at 150.4 99.8) (size 0.5) (drill 0.2) (layers "F.Cu" "B.Cu") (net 3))
 (segment (start 150.5 99.9) (end 154 99.9) (width 0.5) (layer "B.Cu") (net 3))
 (segment (start 150.4 99.8) (end 150.5 99.9) (width 0.5) (layer "B.Cu") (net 3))
 (segment (start 154 99.9) (end 154.5 100.4) (width 0.5) (layer "B.Cu") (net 3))
 (segment (start 149.628 101.428) (end 145.539874 101.428) (width 0.5) (layer "F.Cu") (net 5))
 (segment (start 150.55 102.35) (end 149.628 101.428) (width 0.5) (layer "F.Cu") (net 5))
 (segment (start 144.611874 100.5) (end 142.35 100.5) (width 0.5) (layer "F.Cu") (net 5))
 (segment (start 145.539874 101.428) (end 144.611874 100.5) (width 0.5) (layer "F.Cu") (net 5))
 (segment (start 155.484516 102.35) (end 150.55 102.35) (width 0.5) (layer "F.Cu") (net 5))
 (segment (start 158.65 100.5) (end 157.334516 100.5) (width 0.5) (layer "F.Cu") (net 5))
 (segment (start 157.334516 100.5) (end 155.484516 102.35) (width 0.5) (layer "F.Cu") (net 5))
 (segment (start 158.572 92.528) (end 154.616127 92.528) (width 0.5) (layer "B.Cu") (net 6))
 (segment (start 153.960127 91.872) (end 146.216127 91.872) (width 0.5) (layer "B.Cu") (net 6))
 (segment (start 145.560127 92.528) (end 142.428 92.528) (width 0.5) (layer "B.Cu") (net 6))
 (segment (start 142.428 92.528) (end 142.4 92.5) (width 0.5) (layer "B.Cu") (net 6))
 (segment (start 146.216127 91.872) (end 145.560127 92.528) (width 0.5) (layer "B.Cu") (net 6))
 (segment (start 158.6 92.5) (end 158.572 92.528) (width 0.5) (layer "B.Cu") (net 6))
 (segment (start 154.616127 92.528) (end 153.960127 91.872) (width 0.5) (layer "B.Cu") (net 6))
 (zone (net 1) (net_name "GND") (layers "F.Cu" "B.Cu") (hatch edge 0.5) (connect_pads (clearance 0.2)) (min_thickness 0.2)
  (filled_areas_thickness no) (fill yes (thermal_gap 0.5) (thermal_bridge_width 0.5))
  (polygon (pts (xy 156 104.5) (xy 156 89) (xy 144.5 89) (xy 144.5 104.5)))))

